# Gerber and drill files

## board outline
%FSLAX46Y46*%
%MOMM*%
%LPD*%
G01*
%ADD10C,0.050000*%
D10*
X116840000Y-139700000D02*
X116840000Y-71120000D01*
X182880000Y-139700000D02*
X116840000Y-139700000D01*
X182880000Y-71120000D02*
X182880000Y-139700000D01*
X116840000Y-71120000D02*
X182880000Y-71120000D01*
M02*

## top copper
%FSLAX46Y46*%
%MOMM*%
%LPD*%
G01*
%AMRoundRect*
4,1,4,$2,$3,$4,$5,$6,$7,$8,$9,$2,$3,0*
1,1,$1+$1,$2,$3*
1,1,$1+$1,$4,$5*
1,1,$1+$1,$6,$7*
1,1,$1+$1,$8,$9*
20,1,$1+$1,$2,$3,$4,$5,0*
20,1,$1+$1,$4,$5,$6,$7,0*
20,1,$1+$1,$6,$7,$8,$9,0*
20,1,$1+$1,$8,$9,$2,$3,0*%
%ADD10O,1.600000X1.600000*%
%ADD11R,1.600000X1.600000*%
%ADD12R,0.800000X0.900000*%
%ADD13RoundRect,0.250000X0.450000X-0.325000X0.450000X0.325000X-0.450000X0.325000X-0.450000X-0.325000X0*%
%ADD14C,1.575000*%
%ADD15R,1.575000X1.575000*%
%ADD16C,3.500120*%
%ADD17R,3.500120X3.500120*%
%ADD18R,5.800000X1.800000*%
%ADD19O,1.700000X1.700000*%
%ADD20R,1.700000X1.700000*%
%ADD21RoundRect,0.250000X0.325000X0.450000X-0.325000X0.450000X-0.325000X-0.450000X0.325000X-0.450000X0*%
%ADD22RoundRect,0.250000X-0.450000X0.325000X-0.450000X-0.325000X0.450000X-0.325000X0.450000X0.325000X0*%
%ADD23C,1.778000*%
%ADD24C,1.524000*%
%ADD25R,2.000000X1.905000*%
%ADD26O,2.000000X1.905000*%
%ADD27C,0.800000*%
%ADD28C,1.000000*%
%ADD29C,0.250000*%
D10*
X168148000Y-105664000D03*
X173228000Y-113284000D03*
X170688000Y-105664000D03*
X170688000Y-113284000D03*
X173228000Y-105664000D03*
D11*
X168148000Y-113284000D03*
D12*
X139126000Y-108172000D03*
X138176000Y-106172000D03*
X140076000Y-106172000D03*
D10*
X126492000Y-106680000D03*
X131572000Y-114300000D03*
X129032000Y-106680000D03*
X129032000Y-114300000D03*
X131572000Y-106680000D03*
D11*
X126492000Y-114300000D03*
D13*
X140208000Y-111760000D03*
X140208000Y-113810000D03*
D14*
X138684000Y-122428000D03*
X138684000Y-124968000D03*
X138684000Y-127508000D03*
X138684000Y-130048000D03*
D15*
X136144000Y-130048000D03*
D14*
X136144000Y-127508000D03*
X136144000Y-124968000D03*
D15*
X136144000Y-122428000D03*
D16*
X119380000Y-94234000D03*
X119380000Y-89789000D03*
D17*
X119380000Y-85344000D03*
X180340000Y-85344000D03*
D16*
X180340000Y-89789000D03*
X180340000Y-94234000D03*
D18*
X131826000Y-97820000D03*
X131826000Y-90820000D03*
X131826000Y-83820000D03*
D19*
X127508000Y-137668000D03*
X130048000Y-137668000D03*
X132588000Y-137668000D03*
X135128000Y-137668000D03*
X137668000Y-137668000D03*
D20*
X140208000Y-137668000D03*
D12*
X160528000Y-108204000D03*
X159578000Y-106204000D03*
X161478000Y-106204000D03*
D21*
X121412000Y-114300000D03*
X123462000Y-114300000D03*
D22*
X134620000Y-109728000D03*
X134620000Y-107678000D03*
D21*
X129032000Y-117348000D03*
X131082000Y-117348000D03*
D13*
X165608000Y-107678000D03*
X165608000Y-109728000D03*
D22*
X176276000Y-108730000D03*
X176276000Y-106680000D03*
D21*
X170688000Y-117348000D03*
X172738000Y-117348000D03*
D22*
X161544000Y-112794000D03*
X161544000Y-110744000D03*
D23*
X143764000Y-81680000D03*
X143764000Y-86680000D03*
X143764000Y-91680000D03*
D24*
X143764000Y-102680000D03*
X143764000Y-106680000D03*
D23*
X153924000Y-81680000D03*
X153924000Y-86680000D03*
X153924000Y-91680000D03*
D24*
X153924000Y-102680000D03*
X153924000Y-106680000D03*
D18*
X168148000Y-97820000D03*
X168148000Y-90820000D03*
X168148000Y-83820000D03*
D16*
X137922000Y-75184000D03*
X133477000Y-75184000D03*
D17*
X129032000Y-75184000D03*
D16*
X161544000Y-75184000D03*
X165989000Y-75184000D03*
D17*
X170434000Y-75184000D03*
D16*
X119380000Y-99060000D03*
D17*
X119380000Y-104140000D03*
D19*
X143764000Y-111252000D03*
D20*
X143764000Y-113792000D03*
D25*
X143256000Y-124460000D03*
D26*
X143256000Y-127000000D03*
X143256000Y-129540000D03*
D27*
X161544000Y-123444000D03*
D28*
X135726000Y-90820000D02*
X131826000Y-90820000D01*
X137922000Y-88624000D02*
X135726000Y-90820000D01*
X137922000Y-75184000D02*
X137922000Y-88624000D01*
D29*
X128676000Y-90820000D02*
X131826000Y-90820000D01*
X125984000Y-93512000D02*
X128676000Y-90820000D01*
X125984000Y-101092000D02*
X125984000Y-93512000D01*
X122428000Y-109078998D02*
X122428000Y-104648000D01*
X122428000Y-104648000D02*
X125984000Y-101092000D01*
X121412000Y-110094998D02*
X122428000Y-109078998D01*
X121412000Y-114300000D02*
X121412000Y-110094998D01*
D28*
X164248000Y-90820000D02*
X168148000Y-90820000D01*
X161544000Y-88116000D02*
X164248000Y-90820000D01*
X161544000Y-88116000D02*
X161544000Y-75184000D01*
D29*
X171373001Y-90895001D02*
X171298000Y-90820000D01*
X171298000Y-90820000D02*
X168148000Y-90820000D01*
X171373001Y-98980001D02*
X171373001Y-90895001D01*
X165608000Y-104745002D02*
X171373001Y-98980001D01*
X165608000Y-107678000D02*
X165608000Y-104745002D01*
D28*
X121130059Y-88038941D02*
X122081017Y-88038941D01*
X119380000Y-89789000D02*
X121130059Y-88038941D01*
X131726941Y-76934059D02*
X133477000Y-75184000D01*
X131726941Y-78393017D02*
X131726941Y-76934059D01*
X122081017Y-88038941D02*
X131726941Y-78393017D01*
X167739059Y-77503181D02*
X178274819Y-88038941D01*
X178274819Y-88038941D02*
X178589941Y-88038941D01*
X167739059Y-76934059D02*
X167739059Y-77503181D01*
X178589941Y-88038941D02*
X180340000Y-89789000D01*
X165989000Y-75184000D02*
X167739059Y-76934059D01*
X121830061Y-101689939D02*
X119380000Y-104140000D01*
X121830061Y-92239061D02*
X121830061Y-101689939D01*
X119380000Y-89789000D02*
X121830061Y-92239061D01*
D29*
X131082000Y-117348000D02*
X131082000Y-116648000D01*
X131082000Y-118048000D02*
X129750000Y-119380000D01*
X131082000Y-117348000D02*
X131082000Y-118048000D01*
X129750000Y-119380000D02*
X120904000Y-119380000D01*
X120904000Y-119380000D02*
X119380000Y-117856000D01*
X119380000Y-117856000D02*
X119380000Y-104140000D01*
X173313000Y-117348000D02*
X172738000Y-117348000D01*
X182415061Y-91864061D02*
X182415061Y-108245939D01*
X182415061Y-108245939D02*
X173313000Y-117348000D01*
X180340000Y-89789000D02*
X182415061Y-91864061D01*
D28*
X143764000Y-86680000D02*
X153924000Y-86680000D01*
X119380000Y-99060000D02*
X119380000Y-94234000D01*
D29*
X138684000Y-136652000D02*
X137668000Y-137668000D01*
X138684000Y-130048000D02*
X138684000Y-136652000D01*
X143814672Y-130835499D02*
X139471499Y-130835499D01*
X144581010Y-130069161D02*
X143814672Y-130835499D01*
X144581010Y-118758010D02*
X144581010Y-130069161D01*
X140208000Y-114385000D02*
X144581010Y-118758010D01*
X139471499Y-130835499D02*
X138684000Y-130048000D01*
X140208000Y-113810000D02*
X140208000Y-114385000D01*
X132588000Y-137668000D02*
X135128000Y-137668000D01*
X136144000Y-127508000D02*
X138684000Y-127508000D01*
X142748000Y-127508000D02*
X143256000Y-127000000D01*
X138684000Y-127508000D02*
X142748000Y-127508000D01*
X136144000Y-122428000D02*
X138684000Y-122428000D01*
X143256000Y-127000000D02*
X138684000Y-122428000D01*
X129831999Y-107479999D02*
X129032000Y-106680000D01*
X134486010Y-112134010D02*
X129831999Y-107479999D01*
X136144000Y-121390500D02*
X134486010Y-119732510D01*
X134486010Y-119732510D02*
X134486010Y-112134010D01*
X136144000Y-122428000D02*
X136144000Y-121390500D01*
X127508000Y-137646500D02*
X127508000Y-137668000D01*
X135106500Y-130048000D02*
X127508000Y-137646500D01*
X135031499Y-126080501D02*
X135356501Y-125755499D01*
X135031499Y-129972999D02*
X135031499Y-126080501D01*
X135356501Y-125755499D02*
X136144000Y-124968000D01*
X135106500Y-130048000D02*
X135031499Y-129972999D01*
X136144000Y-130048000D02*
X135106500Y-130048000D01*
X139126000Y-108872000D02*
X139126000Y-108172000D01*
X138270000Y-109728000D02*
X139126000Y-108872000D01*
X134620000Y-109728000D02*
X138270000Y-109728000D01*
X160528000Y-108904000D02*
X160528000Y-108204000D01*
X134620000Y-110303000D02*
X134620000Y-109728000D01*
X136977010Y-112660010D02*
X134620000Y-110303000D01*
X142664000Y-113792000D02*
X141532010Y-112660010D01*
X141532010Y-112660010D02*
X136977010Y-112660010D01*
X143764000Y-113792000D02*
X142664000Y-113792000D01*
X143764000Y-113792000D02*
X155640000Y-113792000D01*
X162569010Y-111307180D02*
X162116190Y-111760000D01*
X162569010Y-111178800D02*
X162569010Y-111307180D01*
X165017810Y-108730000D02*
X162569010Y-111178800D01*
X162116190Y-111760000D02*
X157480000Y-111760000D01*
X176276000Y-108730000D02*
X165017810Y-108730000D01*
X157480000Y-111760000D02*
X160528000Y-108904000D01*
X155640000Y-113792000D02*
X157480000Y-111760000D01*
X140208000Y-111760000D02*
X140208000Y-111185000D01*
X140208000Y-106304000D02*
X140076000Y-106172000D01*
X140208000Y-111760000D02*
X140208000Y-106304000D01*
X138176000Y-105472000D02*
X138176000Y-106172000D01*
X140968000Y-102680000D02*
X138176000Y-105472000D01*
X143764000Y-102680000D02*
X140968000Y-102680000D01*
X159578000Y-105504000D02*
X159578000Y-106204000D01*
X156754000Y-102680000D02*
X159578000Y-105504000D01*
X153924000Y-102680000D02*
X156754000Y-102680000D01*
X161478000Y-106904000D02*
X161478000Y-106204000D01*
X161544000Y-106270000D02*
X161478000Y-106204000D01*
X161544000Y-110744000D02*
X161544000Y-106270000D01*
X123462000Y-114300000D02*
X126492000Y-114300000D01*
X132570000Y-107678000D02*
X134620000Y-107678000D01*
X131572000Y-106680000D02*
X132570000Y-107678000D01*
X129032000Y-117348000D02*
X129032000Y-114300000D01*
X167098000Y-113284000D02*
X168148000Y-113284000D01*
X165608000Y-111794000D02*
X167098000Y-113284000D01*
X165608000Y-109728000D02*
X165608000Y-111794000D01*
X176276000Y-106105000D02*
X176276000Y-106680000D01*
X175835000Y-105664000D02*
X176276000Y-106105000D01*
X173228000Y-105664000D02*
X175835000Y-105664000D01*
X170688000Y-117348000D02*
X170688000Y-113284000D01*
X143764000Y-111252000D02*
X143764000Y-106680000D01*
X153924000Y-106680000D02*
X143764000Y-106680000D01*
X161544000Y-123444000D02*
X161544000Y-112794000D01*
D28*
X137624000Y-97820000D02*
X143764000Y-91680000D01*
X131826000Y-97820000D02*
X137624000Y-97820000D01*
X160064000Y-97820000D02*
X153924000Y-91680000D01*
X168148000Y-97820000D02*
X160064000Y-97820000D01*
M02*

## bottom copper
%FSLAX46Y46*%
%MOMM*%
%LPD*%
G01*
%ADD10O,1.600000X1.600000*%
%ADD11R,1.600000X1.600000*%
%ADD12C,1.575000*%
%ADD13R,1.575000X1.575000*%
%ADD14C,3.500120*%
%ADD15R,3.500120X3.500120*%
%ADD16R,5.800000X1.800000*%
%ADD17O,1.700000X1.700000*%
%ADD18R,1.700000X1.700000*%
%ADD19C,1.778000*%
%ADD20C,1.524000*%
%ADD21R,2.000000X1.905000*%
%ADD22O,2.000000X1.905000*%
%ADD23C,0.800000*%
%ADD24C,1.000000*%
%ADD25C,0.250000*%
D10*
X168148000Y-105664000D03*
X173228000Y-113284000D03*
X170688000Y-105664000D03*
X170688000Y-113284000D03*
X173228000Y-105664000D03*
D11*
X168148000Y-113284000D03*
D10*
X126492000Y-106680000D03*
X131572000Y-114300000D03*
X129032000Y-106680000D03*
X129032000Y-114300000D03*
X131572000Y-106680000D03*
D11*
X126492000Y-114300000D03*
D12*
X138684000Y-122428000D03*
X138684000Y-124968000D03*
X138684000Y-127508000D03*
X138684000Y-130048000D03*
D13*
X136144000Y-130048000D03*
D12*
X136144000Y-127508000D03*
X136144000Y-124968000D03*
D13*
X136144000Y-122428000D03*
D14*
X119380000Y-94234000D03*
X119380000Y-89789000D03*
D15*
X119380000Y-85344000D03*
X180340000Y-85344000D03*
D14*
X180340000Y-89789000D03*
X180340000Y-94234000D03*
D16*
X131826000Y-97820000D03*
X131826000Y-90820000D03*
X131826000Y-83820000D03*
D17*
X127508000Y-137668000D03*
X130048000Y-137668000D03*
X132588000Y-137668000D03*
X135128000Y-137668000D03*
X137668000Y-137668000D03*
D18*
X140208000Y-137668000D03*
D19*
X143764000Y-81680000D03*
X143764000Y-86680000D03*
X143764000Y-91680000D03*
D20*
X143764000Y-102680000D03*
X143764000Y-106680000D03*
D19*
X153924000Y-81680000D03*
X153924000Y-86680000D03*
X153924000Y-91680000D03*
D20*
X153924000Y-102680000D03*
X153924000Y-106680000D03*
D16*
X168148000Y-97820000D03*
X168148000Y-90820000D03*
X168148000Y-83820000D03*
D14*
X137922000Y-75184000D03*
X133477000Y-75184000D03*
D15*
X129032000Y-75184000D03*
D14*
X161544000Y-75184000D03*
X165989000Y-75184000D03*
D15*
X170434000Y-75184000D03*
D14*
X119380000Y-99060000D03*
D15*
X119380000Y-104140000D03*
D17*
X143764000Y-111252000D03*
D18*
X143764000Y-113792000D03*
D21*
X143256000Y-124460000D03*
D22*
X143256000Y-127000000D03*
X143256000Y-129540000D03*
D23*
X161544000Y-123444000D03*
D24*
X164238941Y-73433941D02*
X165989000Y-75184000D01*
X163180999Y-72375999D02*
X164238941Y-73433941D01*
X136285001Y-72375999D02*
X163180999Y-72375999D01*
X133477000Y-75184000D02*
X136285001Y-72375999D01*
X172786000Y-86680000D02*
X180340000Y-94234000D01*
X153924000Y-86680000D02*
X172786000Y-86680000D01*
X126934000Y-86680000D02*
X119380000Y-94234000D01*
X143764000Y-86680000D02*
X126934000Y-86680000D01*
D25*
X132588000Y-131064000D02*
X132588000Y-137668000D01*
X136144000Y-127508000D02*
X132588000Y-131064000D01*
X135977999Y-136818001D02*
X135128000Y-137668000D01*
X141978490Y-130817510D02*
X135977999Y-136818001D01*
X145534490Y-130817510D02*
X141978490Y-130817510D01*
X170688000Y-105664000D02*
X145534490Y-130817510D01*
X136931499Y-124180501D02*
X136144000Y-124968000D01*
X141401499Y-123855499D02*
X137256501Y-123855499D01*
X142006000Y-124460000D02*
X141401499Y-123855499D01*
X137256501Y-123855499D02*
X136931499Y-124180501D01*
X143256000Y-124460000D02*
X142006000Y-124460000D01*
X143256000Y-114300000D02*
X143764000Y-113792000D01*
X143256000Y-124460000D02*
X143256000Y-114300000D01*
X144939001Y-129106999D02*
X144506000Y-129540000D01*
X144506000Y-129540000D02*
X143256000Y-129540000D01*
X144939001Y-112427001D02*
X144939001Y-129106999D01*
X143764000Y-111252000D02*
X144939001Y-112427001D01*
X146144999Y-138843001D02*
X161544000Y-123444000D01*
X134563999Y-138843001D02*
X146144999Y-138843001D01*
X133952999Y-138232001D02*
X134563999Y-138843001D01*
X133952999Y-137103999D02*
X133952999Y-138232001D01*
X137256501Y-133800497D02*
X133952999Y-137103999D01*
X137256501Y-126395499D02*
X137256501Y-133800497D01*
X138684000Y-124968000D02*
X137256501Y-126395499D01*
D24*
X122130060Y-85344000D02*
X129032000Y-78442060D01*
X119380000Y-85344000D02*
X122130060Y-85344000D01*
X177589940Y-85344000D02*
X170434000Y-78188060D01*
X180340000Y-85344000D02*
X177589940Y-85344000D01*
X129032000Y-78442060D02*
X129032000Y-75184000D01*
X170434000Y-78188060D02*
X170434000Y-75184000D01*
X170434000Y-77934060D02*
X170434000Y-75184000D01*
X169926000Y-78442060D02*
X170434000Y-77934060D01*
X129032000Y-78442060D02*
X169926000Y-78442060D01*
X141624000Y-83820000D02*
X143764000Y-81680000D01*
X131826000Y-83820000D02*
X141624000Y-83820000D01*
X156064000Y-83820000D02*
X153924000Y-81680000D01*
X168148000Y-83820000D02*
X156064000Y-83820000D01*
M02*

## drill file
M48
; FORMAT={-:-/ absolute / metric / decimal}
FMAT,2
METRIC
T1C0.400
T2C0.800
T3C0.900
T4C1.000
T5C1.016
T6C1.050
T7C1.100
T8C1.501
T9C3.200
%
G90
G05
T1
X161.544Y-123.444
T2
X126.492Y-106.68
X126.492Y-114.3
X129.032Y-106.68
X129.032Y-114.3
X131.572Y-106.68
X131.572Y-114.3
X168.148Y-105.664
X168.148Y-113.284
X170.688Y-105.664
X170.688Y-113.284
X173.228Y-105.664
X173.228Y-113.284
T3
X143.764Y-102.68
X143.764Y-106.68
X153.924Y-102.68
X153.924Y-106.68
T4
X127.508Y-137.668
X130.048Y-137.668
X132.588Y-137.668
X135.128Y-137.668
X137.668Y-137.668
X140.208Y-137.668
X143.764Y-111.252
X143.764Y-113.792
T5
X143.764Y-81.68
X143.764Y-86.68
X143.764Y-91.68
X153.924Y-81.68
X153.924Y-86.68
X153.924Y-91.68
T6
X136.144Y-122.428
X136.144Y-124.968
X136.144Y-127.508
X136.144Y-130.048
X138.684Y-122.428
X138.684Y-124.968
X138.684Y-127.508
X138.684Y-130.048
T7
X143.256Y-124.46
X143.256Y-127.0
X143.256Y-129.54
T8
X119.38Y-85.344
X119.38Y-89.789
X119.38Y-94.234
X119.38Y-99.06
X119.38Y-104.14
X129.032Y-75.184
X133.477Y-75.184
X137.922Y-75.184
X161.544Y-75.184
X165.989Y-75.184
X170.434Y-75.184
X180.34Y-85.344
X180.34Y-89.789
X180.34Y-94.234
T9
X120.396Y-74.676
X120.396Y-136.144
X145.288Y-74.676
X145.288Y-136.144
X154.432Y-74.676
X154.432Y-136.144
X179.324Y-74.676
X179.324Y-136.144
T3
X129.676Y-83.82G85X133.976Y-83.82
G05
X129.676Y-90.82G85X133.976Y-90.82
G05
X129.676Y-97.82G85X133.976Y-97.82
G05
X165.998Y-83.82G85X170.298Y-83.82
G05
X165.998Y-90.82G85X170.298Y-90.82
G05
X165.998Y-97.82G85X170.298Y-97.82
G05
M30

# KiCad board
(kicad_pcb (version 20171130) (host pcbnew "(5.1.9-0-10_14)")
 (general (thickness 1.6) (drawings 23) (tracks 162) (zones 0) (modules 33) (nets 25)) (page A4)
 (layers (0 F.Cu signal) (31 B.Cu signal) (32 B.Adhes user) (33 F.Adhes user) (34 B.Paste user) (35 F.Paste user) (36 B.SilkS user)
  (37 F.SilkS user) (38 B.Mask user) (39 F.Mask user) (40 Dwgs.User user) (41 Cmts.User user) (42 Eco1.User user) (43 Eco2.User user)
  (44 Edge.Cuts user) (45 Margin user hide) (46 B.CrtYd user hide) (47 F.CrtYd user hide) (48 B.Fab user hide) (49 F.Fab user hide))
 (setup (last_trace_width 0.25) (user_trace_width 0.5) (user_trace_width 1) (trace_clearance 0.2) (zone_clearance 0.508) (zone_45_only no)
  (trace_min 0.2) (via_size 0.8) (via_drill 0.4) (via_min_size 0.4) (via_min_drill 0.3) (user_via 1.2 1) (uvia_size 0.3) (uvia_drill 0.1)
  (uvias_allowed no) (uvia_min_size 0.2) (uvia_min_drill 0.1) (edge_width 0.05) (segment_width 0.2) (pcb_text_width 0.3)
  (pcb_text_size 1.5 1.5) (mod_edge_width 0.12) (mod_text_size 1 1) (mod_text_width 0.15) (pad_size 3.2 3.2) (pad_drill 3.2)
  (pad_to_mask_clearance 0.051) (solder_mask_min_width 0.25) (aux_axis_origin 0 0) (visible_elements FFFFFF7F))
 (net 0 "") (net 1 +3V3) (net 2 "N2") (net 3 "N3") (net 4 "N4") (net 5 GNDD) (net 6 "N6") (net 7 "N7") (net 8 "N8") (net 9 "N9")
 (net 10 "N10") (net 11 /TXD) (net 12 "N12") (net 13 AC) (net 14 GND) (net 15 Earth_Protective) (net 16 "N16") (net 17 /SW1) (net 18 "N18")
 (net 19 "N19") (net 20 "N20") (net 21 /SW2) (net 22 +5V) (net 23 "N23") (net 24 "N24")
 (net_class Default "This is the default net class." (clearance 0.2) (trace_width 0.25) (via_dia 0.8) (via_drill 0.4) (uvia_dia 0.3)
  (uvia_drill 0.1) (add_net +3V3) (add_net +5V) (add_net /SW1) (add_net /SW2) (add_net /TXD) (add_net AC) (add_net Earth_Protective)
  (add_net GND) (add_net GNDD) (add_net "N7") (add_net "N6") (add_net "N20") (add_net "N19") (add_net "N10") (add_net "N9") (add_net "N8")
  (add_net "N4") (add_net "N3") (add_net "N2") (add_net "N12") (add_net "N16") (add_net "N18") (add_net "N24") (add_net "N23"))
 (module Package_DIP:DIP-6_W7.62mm (layer F.Cu) (at 168.148 113.284 90)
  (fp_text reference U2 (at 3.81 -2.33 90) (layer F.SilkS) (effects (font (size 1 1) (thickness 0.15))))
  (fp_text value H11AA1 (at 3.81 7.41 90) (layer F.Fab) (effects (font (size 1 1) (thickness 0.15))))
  (pad 6 thru_hole oval (at 7.62 0 90) (size 1.6 1.6) (drill 0.8) (layers *.Cu *.Mask))
  (pad 3 thru_hole oval (at 0 5.08 90) (size 1.6 1.6) (drill 0.8) (layers *.Cu *.Mask))
  (pad 5 thru_hole oval (at 7.62 2.54 90) (size 1.6 1.6) (drill 0.8) (layers *.Cu *.Mask) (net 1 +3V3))
  (pad 2 thru_hole oval (at 0 2.54 90) (size 1.6 1.6) (drill 0.8) (layers *.Cu *.Mask) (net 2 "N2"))
  (pad 4 thru_hole oval (at 7.62 5.08 90) (size 1.6 1.6) (drill 0.8) (layers *.Cu *.Mask) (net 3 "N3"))
  (pad 1 thru_hole rect (at 0 0 90) (size 1.6 1.6) (drill 0.8) (layers *.Cu *.Mask) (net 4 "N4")))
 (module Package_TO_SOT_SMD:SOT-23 (layer F.Cu) (at 139.126 107.172 270)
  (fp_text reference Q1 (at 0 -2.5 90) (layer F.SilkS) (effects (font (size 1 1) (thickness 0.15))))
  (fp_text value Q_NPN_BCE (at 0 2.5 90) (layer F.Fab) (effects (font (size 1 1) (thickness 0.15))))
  (pad 3 smd rect (at 1 0 270) (size 0.9 0.8) (layers F.Cu F.Paste F.Mask) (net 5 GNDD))
  (pad 2 smd rect (at -1 0.95 270) (size 0.9 0.8) (layers F.Cu F.Paste F.Mask) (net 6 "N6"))
  (pad 1 smd rect (at -1 -0.95 270) (size 0.9 0.8) (layers F.Cu F.Paste F.Mask) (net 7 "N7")))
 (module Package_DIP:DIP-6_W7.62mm (layer F.Cu) (at 126.492 114.3 90)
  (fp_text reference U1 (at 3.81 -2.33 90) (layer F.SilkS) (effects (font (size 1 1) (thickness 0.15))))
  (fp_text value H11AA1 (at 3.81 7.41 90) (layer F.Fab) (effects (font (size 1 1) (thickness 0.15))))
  (pad 6 thru_hole oval (at 7.62 0 90) (size 1.6 1.6) (drill 0.8) (layers *.Cu *.Mask))
  (pad 3 thru_hole oval (at 0 5.08 90) (size 1.6 1.6) (drill 0.8) (layers *.Cu *.Mask))
  (pad 5 thru_hole oval (at 7.62 2.54 90) (size 1.6 1.6) (drill 0.8) (layers *.Cu *.Mask) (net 1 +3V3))
  (pad 2 thru_hole oval (at 0 2.54 90) (size 1.6 1.6) (drill 0.8) (layers *.Cu *.Mask) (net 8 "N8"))
  (pad 4 thru_hole oval (at 7.62 5.08 90) (size 1.6 1.6) (drill 0.8) (layers *.Cu *.Mask) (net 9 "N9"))
  (pad 1 thru_hole rect (at 0 0 90) (size 1.6 1.6) (drill 0.8) (layers *.Cu *.Mask) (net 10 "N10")))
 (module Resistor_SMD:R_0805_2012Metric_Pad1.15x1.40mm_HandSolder (layer F.Cu) (at 140.208 112.785 90)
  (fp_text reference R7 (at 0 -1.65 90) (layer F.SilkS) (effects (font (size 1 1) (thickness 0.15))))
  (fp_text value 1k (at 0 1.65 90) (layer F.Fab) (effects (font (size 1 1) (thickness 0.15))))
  (pad 2 smd roundrect (at 1.025 0 90) (size 1.15 1.4) (layers F.Cu F.Paste F.Mask) (roundrect_rratio 0.217391) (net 7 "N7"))
  (pad 1 smd roundrect (at -1.025 0 90) (size 1.15 1.4) (layers F.Cu F.Paste F.Mask) (roundrect_rratio 0.217391) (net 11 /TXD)))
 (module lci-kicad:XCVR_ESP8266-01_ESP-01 (layer F.Cu) (at 136.144 126.238 180)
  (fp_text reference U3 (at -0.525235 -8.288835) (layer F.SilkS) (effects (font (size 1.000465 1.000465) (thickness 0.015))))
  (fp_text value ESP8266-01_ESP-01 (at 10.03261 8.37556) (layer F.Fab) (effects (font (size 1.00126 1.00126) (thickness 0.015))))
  (pad 8 thru_hole circle (at -2.54 3.81 180) (size 1.575 1.575) (drill 1.05) (layers *.Cu *.Mask) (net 1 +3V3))
  (pad 7 thru_hole circle (at -2.54 1.27 180) (size 1.575 1.575) (drill 1.05) (layers *.Cu *.Mask) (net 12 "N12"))
  (pad 6 thru_hole circle (at -2.54 -1.27 180) (size 1.575 1.575) (drill 1.05) (layers *.Cu *.Mask) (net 1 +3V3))
  (pad 5 thru_hole circle (at -2.54 -3.81 180) (size 1.575 1.575) (drill 1.05) (layers *.Cu *.Mask) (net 11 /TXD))
  (pad 4 thru_hole rect (at 0 -3.81 180) (size 1.575 1.575) (drill 1.05) (layers *.Cu *.Mask) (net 5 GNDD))
  (pad 3 thru_hole circle (at 0 -1.27 180) (size 1.575 1.575) (drill 1.05) (layers *.Cu *.Mask) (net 1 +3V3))
  (pad 2 thru_hole circle (at 0 1.27 180) (size 1.575 1.575) (drill 1.05) (layers *.Cu *.Mask) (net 5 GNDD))
  (pad 1 thru_hole rect (at 0 3.81 180) (size 1.575 1.575) (drill 1.05) (layers *.Cu *.Mask) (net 1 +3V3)))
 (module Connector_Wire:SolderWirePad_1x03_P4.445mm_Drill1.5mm (layer F.Cu) (at 119.38 85.344 270)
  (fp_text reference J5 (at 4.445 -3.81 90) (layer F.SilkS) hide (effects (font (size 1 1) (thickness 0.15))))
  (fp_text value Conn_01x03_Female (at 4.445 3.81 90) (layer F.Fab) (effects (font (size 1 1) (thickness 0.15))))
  (pad 3 thru_hole circle (at 8.89 0 270) (size 3.50012 3.50012) (drill 1.50114) (layers *.Cu *.Mask) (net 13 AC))
  (pad 2 thru_hole circle (at 4.445 0 270) (size 3.50012 3.50012) (drill 1.50114) (layers *.Cu *.Mask) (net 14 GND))
  (pad 1 thru_hole rect (at 0 0 270) (size 3.50012 3.50012) (drill 1.50114) (layers *.Cu *.Mask) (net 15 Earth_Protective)))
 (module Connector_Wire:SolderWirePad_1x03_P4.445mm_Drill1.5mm (layer F.Cu) (at 180.34 85.344 270)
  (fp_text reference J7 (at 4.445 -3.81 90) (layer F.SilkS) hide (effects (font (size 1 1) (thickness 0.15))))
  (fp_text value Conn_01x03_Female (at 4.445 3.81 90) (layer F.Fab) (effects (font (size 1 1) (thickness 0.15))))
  (pad 1 thru_hole rect (at 0 0 270) (size 3.50012 3.50012) (drill 1.50114) (layers *.Cu *.Mask) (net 15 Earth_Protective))
  (pad 2 thru_hole circle (at 4.445 0 270) (size 3.50012 3.50012) (drill 1.50114) (layers *.Cu *.Mask) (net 14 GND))
  (pad 3 thru_hole circle (at 8.89 0 270) (size 3.50012 3.50012) (drill 1.50114) (layers *.Cu *.Mask) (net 13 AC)))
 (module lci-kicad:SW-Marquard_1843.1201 (layer F.Cu) (at 131.572 90.932)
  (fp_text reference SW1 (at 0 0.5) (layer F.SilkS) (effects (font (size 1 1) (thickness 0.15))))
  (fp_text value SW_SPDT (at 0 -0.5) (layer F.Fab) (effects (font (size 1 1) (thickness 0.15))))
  (pad 3 thru_hole rect (at 0.254 6.888) (size 5.8 1.8) (drill oval 5.2 0.9) (layers *.Cu *.Mask) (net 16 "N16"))
  (pad 2 thru_hole rect (at 0.254 -0.112) (size 5.8 1.8) (drill oval 5.2 0.9) (layers *.Cu *.Mask) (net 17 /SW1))
  (pad 1 thru_hole rect (at 0.254 -7.112) (size 5.8 1.8) (drill oval 5.2 0.9) (layers *.Cu *.Mask) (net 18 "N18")))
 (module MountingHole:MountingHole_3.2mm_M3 (layer F.Cu) (at 120.396 74.676)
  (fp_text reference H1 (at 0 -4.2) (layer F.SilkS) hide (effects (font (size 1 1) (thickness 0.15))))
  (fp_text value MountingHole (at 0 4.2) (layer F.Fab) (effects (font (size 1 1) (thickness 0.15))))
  (pad 1 np_thru_hole circle (at 0 0) (size 3.2 3.2) (drill 3.2) (layers *.Cu *.Mask)))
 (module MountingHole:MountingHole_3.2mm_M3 (layer F.Cu) (at 120.396 136.144)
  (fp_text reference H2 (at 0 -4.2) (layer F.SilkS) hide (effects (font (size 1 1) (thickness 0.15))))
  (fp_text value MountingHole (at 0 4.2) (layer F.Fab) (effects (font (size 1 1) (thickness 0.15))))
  (pad 1 np_thru_hole circle (at 0 0) (size 3.2 3.2) (drill 3.2) (layers *.Cu *.Mask)))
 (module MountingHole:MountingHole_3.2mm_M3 (layer F.Cu) (at 179.324 74.676)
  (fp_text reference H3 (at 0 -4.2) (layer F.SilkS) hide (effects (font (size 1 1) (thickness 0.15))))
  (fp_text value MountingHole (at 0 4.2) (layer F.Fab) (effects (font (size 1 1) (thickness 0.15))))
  (pad 1 np_thru_hole circle (at 0 0) (size 3.2 3.2) (drill 3.2) (layers *.Cu *.Mask)))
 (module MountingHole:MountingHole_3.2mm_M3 (layer F.Cu) (at 179.324 136.144)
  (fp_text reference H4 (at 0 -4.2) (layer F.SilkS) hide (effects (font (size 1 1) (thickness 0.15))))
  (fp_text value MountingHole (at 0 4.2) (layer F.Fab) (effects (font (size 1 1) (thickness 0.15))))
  (pad "" np_thru_hole circle (at 0 0) (size 3.2 3.2) (drill 3.2) (layers *.Cu *.Mask)))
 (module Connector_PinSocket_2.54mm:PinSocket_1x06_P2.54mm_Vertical (layer F.Cu) (at 140.208 137.668 270)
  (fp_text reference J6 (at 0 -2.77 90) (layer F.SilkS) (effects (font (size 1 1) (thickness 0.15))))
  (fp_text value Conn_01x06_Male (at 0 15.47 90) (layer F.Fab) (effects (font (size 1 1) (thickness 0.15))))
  (pad 6 thru_hole oval (at 0 12.7 270) (size 1.7 1.7) (drill 1) (layers *.Cu *.Mask) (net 5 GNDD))
  (pad 5 thru_hole oval (at 0 10.16 270) (size 1.7 1.7) (drill 1) (layers *.Cu *.Mask))
  (pad 4 thru_hole oval (at 0 7.62 270) (size 1.7 1.7) (drill 1) (layers *.Cu *.Mask) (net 1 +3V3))
  (pad 3 thru_hole oval (at 0 5.08 270) (size 1.7 1.7) (drill 1) (layers *.Cu *.Mask) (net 1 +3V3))
  (pad 2 thru_hole oval (at 0 2.54 270) (size 1.7 1.7) (drill 1) (layers *.Cu *.Mask) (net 11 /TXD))
  (pad 1 thru_hole rect (at 0 0 270) (size 1.7 1.7) (drill 1) (layers *.Cu *.Mask)))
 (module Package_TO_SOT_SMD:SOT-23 (layer F.Cu) (at 160.528 107.204 270)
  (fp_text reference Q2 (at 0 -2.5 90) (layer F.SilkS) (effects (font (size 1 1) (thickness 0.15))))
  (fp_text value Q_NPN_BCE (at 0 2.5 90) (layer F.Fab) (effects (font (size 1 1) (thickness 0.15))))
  (pad 3 smd rect (at 1 0 270) (size 0.9 0.8) (layers F.Cu F.Paste F.Mask) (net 5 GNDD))
  (pad 2 smd rect (at -1 0.95 270) (size 0.9 0.8) (layers F.Cu F.Paste F.Mask) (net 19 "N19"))
  (pad 1 smd rect (at -1 -0.95 270) (size 0.9 0.8) (layers F.Cu F.Paste F.Mask) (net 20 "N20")))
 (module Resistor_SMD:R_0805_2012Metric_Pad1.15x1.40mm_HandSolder (layer F.Cu) (at 122.437 114.3 180)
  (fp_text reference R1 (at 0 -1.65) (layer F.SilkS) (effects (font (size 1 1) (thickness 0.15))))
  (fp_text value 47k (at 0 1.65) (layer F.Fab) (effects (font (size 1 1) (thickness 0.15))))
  (pad 2 smd roundrect (at 1.025 0 180) (size 1.15 1.4) (layers F.Cu F.Paste F.Mask) (roundrect_rratio 0.217391) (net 17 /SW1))
  (pad 1 smd roundrect (at -1.025 0 180) (size 1.15 1.4) (layers F.Cu F.Paste F.Mask) (roundrect_rratio 0.217391) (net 10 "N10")))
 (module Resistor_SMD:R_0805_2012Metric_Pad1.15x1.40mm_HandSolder (layer F.Cu) (at 134.62 108.703 270)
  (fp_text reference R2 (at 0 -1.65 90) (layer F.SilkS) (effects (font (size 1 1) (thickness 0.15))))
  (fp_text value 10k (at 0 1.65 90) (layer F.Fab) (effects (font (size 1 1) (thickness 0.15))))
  (pad 2 smd roundrect (at 1.025 0 270) (size 1.15 1.4) (layers F.Cu F.Paste F.Mask) (roundrect_rratio 0.217391) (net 5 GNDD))
  (pad 1 smd roundrect (at -1.025 0 270) (size 1.15 1.4) (layers F.Cu F.Paste F.Mask) (roundrect_rratio 0.217391) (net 9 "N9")))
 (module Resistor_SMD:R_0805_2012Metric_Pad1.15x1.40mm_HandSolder (layer F.Cu) (at 130.057 117.348 180)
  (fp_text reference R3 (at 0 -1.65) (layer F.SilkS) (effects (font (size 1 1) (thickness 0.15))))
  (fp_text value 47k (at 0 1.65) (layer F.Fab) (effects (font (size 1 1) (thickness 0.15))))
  (pad 2 smd roundrect (at 1.025 0 180) (size 1.15 1.4) (layers F.Cu F.Paste F.Mask) (roundrect_rratio 0.217391) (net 8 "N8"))
  (pad 1 smd roundrect (at -1.025 0 180) (size 1.15 1.4) (layers F.Cu F.Paste F.Mask) (roundrect_rratio 0.217391) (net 14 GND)))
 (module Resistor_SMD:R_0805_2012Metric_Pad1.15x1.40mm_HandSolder (layer F.Cu) (at 165.608 108.703 90)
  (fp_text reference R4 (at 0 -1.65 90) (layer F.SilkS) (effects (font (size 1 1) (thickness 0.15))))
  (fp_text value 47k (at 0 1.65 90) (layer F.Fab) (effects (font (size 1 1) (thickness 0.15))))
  (pad 2 smd roundrect (at 1.025 0 90) (size 1.15 1.4) (layers F.Cu F.Paste F.Mask) (roundrect_rratio 0.217391) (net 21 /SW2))
  (pad 1 smd roundrect (at -1.025 0 90) (size 1.15 1.4) (layers F.Cu F.Paste F.Mask) (roundrect_rratio 0.217391) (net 4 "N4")))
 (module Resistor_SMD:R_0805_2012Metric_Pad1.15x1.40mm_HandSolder (layer F.Cu) (at 176.276 107.705 270)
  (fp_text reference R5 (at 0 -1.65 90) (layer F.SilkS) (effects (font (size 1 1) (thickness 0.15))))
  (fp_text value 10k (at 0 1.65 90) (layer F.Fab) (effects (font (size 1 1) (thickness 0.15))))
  (pad 2 smd roundrect (at 1.025 0 270) (size 1.15 1.4) (layers F.Cu F.Paste F.Mask) (roundrect_rratio 0.217391) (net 5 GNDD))
  (pad 1 smd roundrect (at -1.025 0 270) (size 1.15 1.4) (layers F.Cu F.Paste F.Mask) (roundrect_rratio 0.217391) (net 3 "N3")))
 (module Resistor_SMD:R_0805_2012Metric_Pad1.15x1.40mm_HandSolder (layer F.Cu) (at 171.713 117.348 180)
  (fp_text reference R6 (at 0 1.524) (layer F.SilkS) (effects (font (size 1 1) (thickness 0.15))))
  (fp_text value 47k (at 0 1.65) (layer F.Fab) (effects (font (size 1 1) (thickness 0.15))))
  (pad 2 smd roundrect (at 1.025 0 180) (size 1.15 1.4) (layers F.Cu F.Paste F.Mask) (roundrect_rratio 0.217391) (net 2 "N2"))
  (pad 1 smd roundrect (at -1.025 0 180) (size 1.15 1.4) (layers F.Cu F.Paste F.Mask) (roundrect_rratio 0.217391) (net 14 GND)))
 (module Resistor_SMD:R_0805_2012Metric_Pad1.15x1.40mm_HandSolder (layer F.Cu) (at 161.544 111.769 270)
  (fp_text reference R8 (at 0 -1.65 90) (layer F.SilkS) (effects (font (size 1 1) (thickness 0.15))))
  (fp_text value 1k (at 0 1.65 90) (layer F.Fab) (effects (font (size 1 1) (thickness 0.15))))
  (pad 2 smd roundrect (at 1.025 0 270) (size 1.15 1.4) (layers F.Cu F.Paste F.Mask) (roundrect_rratio 0.217391) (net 12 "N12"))
  (pad 1 smd roundrect (at -1.025 0 270) (size 1.15 1.4) (layers F.Cu F.Paste F.Mask) (roundrect_rratio 0.217391) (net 20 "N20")))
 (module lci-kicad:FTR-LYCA (layer F.Cu) (at 143.764 106.68 90)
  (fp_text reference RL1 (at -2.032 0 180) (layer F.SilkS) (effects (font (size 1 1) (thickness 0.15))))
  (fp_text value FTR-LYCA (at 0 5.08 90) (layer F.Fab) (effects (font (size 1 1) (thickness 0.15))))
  (pad 5 thru_hole circle (at 25 0 90) (size 1.778 1.778) (drill 1.016) (layers *.Cu *.Mask) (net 18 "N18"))
  (pad 4 thru_hole circle (at 20 0 90) (size 1.778 1.778) (drill 1.016) (layers *.Cu *.Mask) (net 13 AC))
  (pad 3 thru_hole circle (at 15 0 90) (size 1.778 1.778) (drill 1.016) (layers *.Cu *.Mask) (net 16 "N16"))
  (pad 2 thru_hole circle (at 4 0 90) (size 1.524 1.524) (drill 0.9) (layers *.Cu *.Mask) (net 6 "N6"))
  (pad 1 thru_hole circle (at 0 0 90) (size 1.524 1.524) (drill 0.9) (layers *.Cu *.Mask) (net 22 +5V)))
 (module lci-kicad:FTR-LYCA (layer F.Cu) (at 153.924 106.68 90)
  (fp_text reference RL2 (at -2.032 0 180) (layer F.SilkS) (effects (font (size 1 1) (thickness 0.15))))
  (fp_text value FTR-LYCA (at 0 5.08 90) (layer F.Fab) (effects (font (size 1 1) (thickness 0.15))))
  (pad 5 thru_hole circle (at 25 0 90) (size 1.778 1.778) (drill 1.016) (layers *.Cu *.Mask) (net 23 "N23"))
  (pad 4 thru_hole circle (at 20 0 90) (size 1.778 1.778) (drill 1.016) (layers *.Cu *.Mask) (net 13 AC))
  (pad 3 thru_hole circle (at 15 0 90) (size 1.778 1.778) (drill 1.016) (layers *.Cu *.Mask) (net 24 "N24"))
  (pad 2 thru_hole circle (at 4 0 90) (size 1.524 1.524) (drill 0.9) (layers *.Cu *.Mask) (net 19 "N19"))
  (pad 1 thru_hole circle (at 0 0 90) (size 1.524 1.524) (drill 0.9) (layers *.Cu *.Mask) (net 22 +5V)))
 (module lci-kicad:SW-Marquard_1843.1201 (layer F.Cu) (at 167.894 90.932)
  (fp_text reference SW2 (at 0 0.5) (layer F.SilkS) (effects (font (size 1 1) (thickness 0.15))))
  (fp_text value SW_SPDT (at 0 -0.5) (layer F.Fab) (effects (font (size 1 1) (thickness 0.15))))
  (pad 3 thru_hole rect (at 0.254 6.888) (size 5.8 1.8) (drill oval 5.2 0.9) (layers *.Cu *.Mask) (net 24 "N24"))
  (pad 2 thru_hole rect (at 0.254 -0.112) (size 5.8 1.8) (drill oval 5.2 0.9) (layers *.Cu *.Mask) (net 21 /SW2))
  (pad 1 thru_hole rect (at 0.254 -7.112) (size 5.8 1.8) (drill oval 5.2 0.9) (layers *.Cu *.Mask) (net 23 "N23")))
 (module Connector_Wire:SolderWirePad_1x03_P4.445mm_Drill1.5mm (layer F.Cu) (at 129.032 75.184)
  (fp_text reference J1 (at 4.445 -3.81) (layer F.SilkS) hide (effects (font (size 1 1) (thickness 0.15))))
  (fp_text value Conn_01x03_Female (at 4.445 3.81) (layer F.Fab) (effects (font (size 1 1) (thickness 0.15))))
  (pad 3 thru_hole circle (at 8.89 0) (size 3.50012 3.50012) (drill 1.50114) (layers *.Cu *.Mask) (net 17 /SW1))
  (pad 2 thru_hole circle (at 4.445 0) (size 3.50012 3.50012) (drill 1.50114) (layers *.Cu *.Mask) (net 14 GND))
  (pad 1 thru_hole rect (at 0 0) (size 3.50012 3.50012) (drill 1.50114) (layers *.Cu *.Mask) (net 15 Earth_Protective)))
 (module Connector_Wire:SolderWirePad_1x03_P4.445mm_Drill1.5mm (layer F.Cu) (at 170.434 75.184 180)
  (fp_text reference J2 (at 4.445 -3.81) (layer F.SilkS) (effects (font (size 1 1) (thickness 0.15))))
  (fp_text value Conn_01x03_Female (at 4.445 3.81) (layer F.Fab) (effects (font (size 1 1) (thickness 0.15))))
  (pad 3 thru_hole circle (at 8.89 0 180) (size 3.50012 3.50012) (drill 1.50114) (layers *.Cu *.Mask) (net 21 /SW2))
  (pad 2 thru_hole circle (at 4.445 0 180) (size 3.50012 3.50012) (drill 1.50114) (layers *.Cu *.Mask) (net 14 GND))
  (pad 1 thru_hole rect (at 0 0 180) (size 3.50012 3.50012) (drill 1.50114) (layers *.Cu *.Mask) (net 15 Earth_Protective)))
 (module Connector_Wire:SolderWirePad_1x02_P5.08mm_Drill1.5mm (layer F.Cu) (at 119.38 104.14 90)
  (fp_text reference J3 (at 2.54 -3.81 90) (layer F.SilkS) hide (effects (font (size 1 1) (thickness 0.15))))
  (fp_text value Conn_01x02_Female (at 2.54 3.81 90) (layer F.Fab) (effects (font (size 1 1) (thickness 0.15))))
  (pad 2 thru_hole circle (at 5.08 0 90) (size 3.50012 3.50012) (drill 1.50114) (layers *.Cu *.Mask) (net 13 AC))
  (pad 1 thru_hole rect (at 0 0 90) (size 3.50012 3.50012) (drill 1.50114) (layers *.Cu *.Mask) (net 14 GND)))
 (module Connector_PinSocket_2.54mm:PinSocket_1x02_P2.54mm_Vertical (layer F.Cu) (at 143.764 113.792 180)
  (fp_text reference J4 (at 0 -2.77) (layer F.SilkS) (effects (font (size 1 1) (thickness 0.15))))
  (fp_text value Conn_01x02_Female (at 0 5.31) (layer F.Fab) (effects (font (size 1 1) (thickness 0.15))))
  (pad 2 thru_hole oval (at 0 2.54 180) (size 1.7 1.7) (drill 1) (layers *.Cu *.Mask) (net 22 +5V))
  (pad 1 thru_hole rect (at 0 0 180) (size 1.7 1.7) (drill 1) (layers *.Cu *.Mask) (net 5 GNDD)))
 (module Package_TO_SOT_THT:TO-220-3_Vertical (layer F.Cu) (at 143.256 124.46 270)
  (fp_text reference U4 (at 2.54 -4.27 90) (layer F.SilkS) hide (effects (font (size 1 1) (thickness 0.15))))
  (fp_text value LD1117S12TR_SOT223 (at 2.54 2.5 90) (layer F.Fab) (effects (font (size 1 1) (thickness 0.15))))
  (pad 1 thru_hole rect (at 0 0 270) (size 1.905 2) (drill 1.1) (layers *.Cu *.Mask) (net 5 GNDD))
  (pad 2 thru_hole oval (at 2.54 0 270) (size 1.905 2) (drill 1.1) (layers *.Cu *.Mask) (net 1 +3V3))
  (pad 3 thru_hole oval (at 5.08 0 270) (size 1.905 2) (drill 1.1) (layers *.Cu *.Mask) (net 22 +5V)))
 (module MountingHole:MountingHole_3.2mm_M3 (layer F.Cu) (at 145.288 74.676)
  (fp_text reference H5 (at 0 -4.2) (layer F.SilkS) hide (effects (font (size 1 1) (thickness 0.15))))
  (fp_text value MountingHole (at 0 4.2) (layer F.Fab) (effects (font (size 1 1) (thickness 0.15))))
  (pad 1 np_thru_hole circle (at 0 0) (size 3.2 3.2) (drill 3.2) (layers *.Cu *.Mask)))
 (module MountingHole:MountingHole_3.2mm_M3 (layer F.Cu) (at 154.432 74.676)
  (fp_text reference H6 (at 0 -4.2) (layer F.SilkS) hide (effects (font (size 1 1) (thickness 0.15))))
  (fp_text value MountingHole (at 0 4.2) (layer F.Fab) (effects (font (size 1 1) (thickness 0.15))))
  (pad 1 np_thru_hole circle (at 0 0) (size 3.2 3.2) (drill 3.2) (layers *.Cu *.Mask)))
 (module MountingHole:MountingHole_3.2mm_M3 (layer F.Cu) (at 145.288 136.144)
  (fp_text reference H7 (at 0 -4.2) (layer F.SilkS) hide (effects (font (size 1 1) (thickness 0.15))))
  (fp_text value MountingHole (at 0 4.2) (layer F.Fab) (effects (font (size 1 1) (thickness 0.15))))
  (pad 1 np_thru_hole circle (at 0 0) (size 3.2 3.2) (drill 3.2) (layers *.Cu *.Mask)))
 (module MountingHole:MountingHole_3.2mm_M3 (layer F.Cu) (at 154.432 136.144)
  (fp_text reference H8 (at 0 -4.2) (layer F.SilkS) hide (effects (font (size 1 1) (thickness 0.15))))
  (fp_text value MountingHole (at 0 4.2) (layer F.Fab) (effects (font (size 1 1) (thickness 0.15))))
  (pad 1 np_thru_hole circle (at 0 0) (size 3.2 3.2) (drill 3.2) (layers *.Cu *.Mask)))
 (gr_line (start 116.84 139.7) (end 116.84 71.12) (layer Edge.Cuts) (width 0.05))
 (gr_line (start 182.88 139.7) (end 116.84 139.7) (layer Edge.Cuts) (width 0.05))
 (gr_line (start 182.88 71.12) (end 182.88 139.7) (layer Edge.Cuts) (width 0.05))
 (gr_line (start 116.84 71.12) (end 182.88 71.12) (layer Edge.Cuts) (width 0.05))
 (segment (start 135.726 90.82) (end 131.826 90.82) (width 1) (layer F.Cu) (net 17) (status 20))
 (segment (start 137.922 88.624) (end 135.726 90.82) (width 1) (layer F.Cu) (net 17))
 (segment (start 137.922 75.184) (end 137.922 88.624) (width 1) (layer F.Cu) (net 17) (status 10))
 (segment (start 128.676 90.82) (end 131.826 90.82) (width 0.25) (layer F.Cu) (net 17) (status 20))
 (segment (start 125.984 93.512) (end 128.676 90.82) (width 0.25) (layer F.Cu) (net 17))
 (segment (start 125.984 101.092) (end 125.984 93.512) (width 0.25) (layer F.Cu) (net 17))
 (segment (start 122.428 109.078998) (end 122.428 104.648) (width 0.25) (layer F.Cu) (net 17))
 (segment (start 122.428 104.648) (end 125.984 101.092) (width 0.25) (layer F.Cu) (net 17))
 (segment (start 121.412 110.094998) (end 122.428 109.078998) (width 0.25) (layer F.Cu) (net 17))
 (segment (start 121.412 114.3) (end 121.412 110.094998) (width 0.25) (layer F.Cu) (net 17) (status 10))
 (segment (start 164.248 90.82) (end 168.148 90.82) (width 1) (layer F.Cu) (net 21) (status 20))
 (segment (start 161.544 88.116) (end 164.248 90.82) (width 1) (layer F.Cu) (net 21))
 (segment (start 161.544 88.116) (end 161.544 75.184) (width 1) (layer F.Cu) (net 21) (status 20))
 (segment (start 171.373001 90.895001) (end 171.298 90.82) (width 0.25) (layer F.Cu) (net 21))
 (segment (start 171.298 90.82) (end 168.148 90.82) (width 0.25) (layer F.Cu) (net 21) (status 20))
 (segment (start 171.373001 98.980001) (end 171.373001 90.895001) (width 0.25) (layer F.Cu) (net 21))
 (segment (start 165.608 104.745002) (end 171.373001 98.980001) (width 0.25) (layer F.Cu) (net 21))
 (segment (start 165.608 107.678) (end 165.608 104.745002) (width 0.25) (layer F.Cu) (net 21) (status 10))
 (segment (start 121.130059 88.038941) (end 122.081017 88.038941) (width 1) (layer F.Cu) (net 14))
 (segment (start 119.38 89.789) (end 121.130059 88.038941) (width 1) (layer F.Cu) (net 14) (status 10))
 (segment (start 164.238941 73.433941) (end 165.989 75.184) (width 1) (layer B.Cu) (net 14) (status 20))
 (segment (start 163.180999 72.375999) (end 164.238941 73.433941) (width 1) (layer B.Cu) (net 14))
 (segment (start 136.285001 72.375999) (end 163.180999 72.375999) (width 1) (layer B.Cu) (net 14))
 (segment (start 133.477 75.184) (end 136.285001 72.375999) (width 1) (layer B.Cu) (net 14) (status 10))
 (segment (start 131.726941 76.934059) (end 133.477 75.184) (width 1) (layer F.Cu) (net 14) (status 20))
 (segment (start 131.726941 78.393017) (end 131.726941 76.934059) (width 1) (layer F.Cu) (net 14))
 (segment (start 122.081017 88.038941) (end 131.726941 78.393017) (width 1) (layer F.Cu) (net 14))
 (segment (start 167.739059 77.503181) (end 178.274819 88.038941) (width 1) (layer F.Cu) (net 14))
 (segment (start 178.274819 88.038941) (end 178.589941 88.038941) (width 1) (layer F.Cu) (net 14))
 (segment (start 167.739059 76.934059) (end 167.739059 77.503181) (width 1) (layer F.Cu) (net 14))
 (segment (start 178.589941 88.038941) (end 180.34 89.789) (width 1) (layer F.Cu) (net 14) (status 20))
 (segment (start 165.989 75.184) (end 167.739059 76.934059) (width 1) (layer F.Cu) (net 14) (status 10))
 (segment (start 121.830061 101.689939) (end 119.38 104.14) (width 1) (layer F.Cu) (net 14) (status 20))
 (segment (start 121.830061 92.239061) (end 121.830061 101.689939) (width 1) (layer F.Cu) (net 14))
 (segment (start 119.38 89.789) (end 121.830061 92.239061) (width 1) (layer F.Cu) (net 14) (status 10))
 (segment (start 131.082 117.348) (end 131.082 116.648) (width 0.25) (layer F.Cu) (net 14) (status 30))
 (segment (start 131.082 118.048) (end 129.75 119.38) (width 0.25) (layer F.Cu) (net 14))
 (segment (start 131.082 117.348) (end 131.082 118.048) (width 0.25) (layer F.Cu) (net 14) (status 10))
 (segment (start 129.75 119.38) (end 120.904 119.38) (width 0.25) (layer F.Cu) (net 14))
 (segment (start 120.904 119.38) (end 119.38 117.856) (width 0.25) (layer F.Cu) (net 14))
 (segment (start 119.38 117.856) (end 119.38 104.14) (width 0.25) (layer F.Cu) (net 14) (status 20))
 (segment (start 173.313 117.348) (end 172.738 117.348) (width 0.25) (layer F.Cu) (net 14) (status 20))
 (segment (start 182.415061 91.864061) (end 182.415061 108.245939) (width 0.25) (layer F.Cu) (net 14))
 (segment (start 182.415061 108.245939) (end 173.313 117.348) (width 0.25) (layer F.Cu) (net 14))
 (segment (start 180.34 89.789) (end 182.415061 91.864061) (width 0.25) (layer F.Cu) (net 14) (status 10))
 (segment (start 143.764 86.68) (end 153.924 86.68) (width 1) (layer F.Cu) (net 13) (status 30))
 (segment (start 119.38 99.06) (end 119.38 94.234) (width 1) (layer F.Cu) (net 13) (status 30))
 (segment (start 172.786 86.68) (end 180.34 94.234) (width 1) (layer B.Cu) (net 13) (status 20))
 (segment (start 153.924 86.68) (end 172.786 86.68) (width 1) (layer B.Cu) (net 13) (status 10))
 (segment (start 126.934 86.68) (end 119.38 94.234) (width 1) (layer B.Cu) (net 13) (status 20))
 (segment (start 143.764 86.68) (end 126.934 86.68) (width 1) (layer B.Cu) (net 13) (status 10))
 (segment (start 138.684 136.652) (end 137.668 137.668) (width 0.25) (layer F.Cu) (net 11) (status 20))
 (segment (start 138.684 130.048) (end 138.684 136.652) (width 0.25) (layer F.Cu) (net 11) (status 10))
 (segment (start 143.814672 130.835499) (end 139.471499 130.835499) (width 0.25) (layer F.Cu) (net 11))
 (segment (start 144.58101 130.069161) (end 143.814672 130.835499) (width 0.25) (layer F.Cu) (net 11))
 (segment (start 144.58101 118.75801) (end 144.58101 130.069161) (width 0.25) (layer F.Cu) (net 11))
 (segment (start 140.208 114.385) (end 144.58101 118.75801) (width 0.25) (layer F.Cu) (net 11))
 (segment (start 139.471499 130.835499) (end 138.684 130.048) (width 0.25) (layer F.Cu) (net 11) (status 20))
 (segment (start 140.208 113.81) (end 140.208 114.385) (width 0.25) (layer F.Cu) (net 11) (status 10))
 (segment (start 132.588 137.668) (end 135.128 137.668) (width 0.25) (layer F.Cu) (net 1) (status 30))
 (segment (start 136.144 127.508) (end 138.684 127.508) (width 0.25) (layer F.Cu) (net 1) (status 30))
 (segment (start 142.748 127.508) (end 143.256 127) (width 0.25) (layer F.Cu) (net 1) (status 30))
 (segment (start 138.684 127.508) (end 142.748 127.508) (width 0.25) (layer F.Cu) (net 1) (status 30))
 (segment (start 136.144 122.428) (end 138.684 122.428) (width 0.25) (layer F.Cu) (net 1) (status 30))
 (segment (start 143.256 127) (end 138.684 122.428) (width 0.25) (layer F.Cu) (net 1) (status 30))
 (segment (start 132.588 131.064) (end 132.588 137.668) (width 0.25) (layer B.Cu) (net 1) (status 20))
 (segment (start 136.144 127.508) (end 132.588 131.064) (width 0.25) (layer B.Cu) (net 1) (status 10))
 (segment (start 129.831999 107.479999) (end 129.032 106.68) (width 0.25) (layer F.Cu) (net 1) (status 20))
 (segment (start 134.48601 112.13401) (end 129.831999 107.479999) (width 0.25) (layer F.Cu) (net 1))
 (segment (start 136.144 121.3905) (end 134.48601 119.73251) (width 0.25) (layer F.Cu) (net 1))
 (segment (start 134.48601 119.73251) (end 134.48601 112.13401) (width 0.25) (layer F.Cu) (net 1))
 (segment (start 136.144 122.428) (end 136.144 121.3905) (width 0.25) (layer F.Cu) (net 1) (status 10))
 (segment (start 135.977999 136.818001) (end 135.128 137.668) (width 0.25) (layer B.Cu) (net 1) (status 20))
 (segment (start 141.97849 130.81751) (end 135.977999 136.818001) (width 0.25) (layer B.Cu) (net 1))
 (segment (start 145.53449 130.81751) (end 141.97849 130.81751) (width 0.25) (layer B.Cu) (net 1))
 (segment (start 170.688 105.664) (end 145.53449 130.81751) (width 0.25) (layer B.Cu) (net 1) (status 10))
 (segment (start 127.508 137.6465) (end 127.508 137.668) (width 0.25) (layer F.Cu) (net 5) (status 30))
 (segment (start 135.1065 130.048) (end 127.508 137.6465) (width 0.25) (layer F.Cu) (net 5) (status 20))
 (segment (start 135.031499 126.080501) (end 135.356501 125.755499) (width 0.25) (layer F.Cu) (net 5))
 (segment (start 135.031499 129.972999) (end 135.031499 126.080501) (width 0.25) (layer F.Cu) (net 5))
 (segment (start 135.356501 125.755499) (end 136.144 124.968) (width 0.25) (layer F.Cu) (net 5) (status 20))
 (segment (start 135.1065 130.048) (end 135.031499 129.972999) (width 0.25) (layer F.Cu) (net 5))
 (segment (start 136.144 130.048) (end 135.1065 130.048) (width 0.25) (layer F.Cu) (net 5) (status 10))
 (segment (start 139.126 108.872) (end 139.126 108.172) (width 0.25) (layer F.Cu) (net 5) (status 20))
 (segment (start 138.27 109.728) (end 139.126 108.872) (width 0.25) (layer F.Cu) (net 5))
 (segment (start 134.62 109.728) (end 138.27 109.728) (width 0.25) (layer F.Cu) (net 5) (status 10))
 (segment (start 136.931499 124.180501) (end 136.144 124.968) (width 0.25) (layer B.Cu) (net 5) (status 20))
 (segment (start 141.401499 123.855499) (end 137.256501 123.855499) (width 0.25) (layer B.Cu) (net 5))
 (segment (start 142.006 124.46) (end 141.401499 123.855499) (width 0.25) (layer B.Cu) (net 5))
 (segment (start 137.256501 123.855499) (end 136.931499 124.180501) (width 0.25) (layer B.Cu) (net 5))
 (segment (start 143.256 124.46) (end 142.006 124.46) (width 0.25) (layer B.Cu) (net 5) (status 10))
 (segment (start 143.256 114.3) (end 143.764 113.792) (width 0.25) (layer B.Cu) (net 5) (status 30))
 (segment (start 143.256 124.46) (end 143.256 114.3) (width 0.25) (layer B.Cu) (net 5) (status 30))
 (segment (start 160.528 108.904) (end 160.528 108.204) (width 0.25) (layer F.Cu) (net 5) (status 20))
 (segment (start 134.62 110.303) (end 134.62 109.728) (width 0.25) (layer F.Cu) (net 5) (status 20))
 (segment (start 136.97701 112.66001) (end 134.62 110.303) (width 0.25) (layer F.Cu) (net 5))
 (segment (start 142.664 113.792) (end 141.53201 112.66001) (width 0.25) (layer F.Cu) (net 5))
 (segment (start 141.53201 112.66001) (end 136.97701 112.66001) (width 0.25) (layer F.Cu) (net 5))
 (segment (start 143.764 113.792) (end 142.664 113.792) (width 0.25) (layer F.Cu) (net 5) (status 10))
 (segment (start 143.764 113.792) (end 155.64 113.792) (width 0.25) (layer F.Cu) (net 5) (status 10))
 (segment (start 162.56901 111.30718) (end 162.11619 111.76) (width 0.25) (layer F.Cu) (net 5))
 (segment (start 162.56901 111.1788) (end 162.56901 111.30718) (width 0.25) (layer F.Cu) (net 5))
 (segment (start 165.01781 108.73) (end 162.56901 111.1788) (width 0.25) (layer F.Cu) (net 5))
 (segment (start 162.11619 111.76) (end 157.48 111.76) (width 0.25) (layer F.Cu) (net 5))
 (segment (start 176.276 108.73) (end 165.01781 108.73) (width 0.25) (layer F.Cu) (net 5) (status 10))
 (segment (start 157.48 111.76) (end 160.528 108.904) (width 0.25) (layer F.Cu) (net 5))
 (segment (start 155.64 113.792) (end 157.48 111.76) (width 0.25) (layer F.Cu) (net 5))
 (segment (start 140.208 111.76) (end 140.208 111.185) (width 0.25) (layer F.Cu) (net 7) (status 30))
 (segment (start 140.208 106.304) (end 140.076 106.172) (width 0.25) (layer F.Cu) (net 7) (status 30))
 (segment (start 140.208 111.76) (end 140.208 106.304) (width 0.25) (layer F.Cu) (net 7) (status 30))
 (segment (start 138.176 105.472) (end 138.176 106.172) (width 0.25) (layer F.Cu) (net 6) (status 20))
 (segment (start 140.968 102.68) (end 138.176 105.472) (width 0.25) (layer F.Cu) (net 6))
 (segment (start 143.764 102.68) (end 140.968 102.68) (width 0.25) (layer F.Cu) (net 6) (status 10))
 (segment (start 159.578 105.504) (end 159.578 106.204) (width 0.25) (layer F.Cu) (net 19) (status 20))
 (segment (start 156.754 102.68) (end 159.578 105.504) (width 0.25) (layer F.Cu) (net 19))
 (segment (start 153.924 102.68) (end 156.754 102.68) (width 0.25) (layer F.Cu) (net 19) (status 10))
 (segment (start 161.478 106.904) (end 161.478 106.204) (width 0.25) (layer F.Cu) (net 20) (status 20))
 (segment (start 161.544 106.27) (end 161.478 106.204) (width 0.25) (layer F.Cu) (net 20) (status 30))
 (segment (start 161.544 110.744) (end 161.544 106.27) (width 0.25) (layer F.Cu) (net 20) (status 30))
 (segment (start 123.462 114.3) (end 126.492 114.3) (width 0.25) (layer F.Cu) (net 10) (status 30))
 (segment (start 132.57 107.678) (end 134.62 107.678) (width 0.25) (layer F.Cu) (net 9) (status 20))
 (segment (start 131.572 106.68) (end 132.57 107.678) (width 0.25) (layer F.Cu) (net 9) (status 10))
 (segment (start 129.032 117.348) (end 129.032 114.3) (width 0.25) (layer F.Cu) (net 8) (status 30))
 (segment (start 167.098 113.284) (end 168.148 113.284) (width 0.25) (layer F.Cu) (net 4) (status 20))
 (segment (start 165.608 111.794) (end 167.098 113.284) (width 0.25) (layer F.Cu) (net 4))
 (segment (start 165.608 109.728) (end 165.608 111.794) (width 0.25) (layer F.Cu) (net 4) (status 10))
 (segment (start 176.276 106.105) (end 176.276 106.68) (width 0.25) (layer F.Cu) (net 3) (status 30))
 (segment (start 175.835 105.664) (end 176.276 106.105) (width 0.25) (layer F.Cu) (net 3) (status 20))
 (segment (start 173.228 105.664) (end 175.835 105.664) (width 0.25) (layer F.Cu) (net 3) (status 10))
 (segment (start 170.688 117.348) (end 170.688 113.284) (width 0.25) (layer F.Cu) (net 2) (status 30))
 (segment (start 143.764 111.252) (end 143.764 106.68) (width 0.25) (layer F.Cu) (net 22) (status 30))
 (segment (start 153.924 106.68) (end 143.764 106.68) (width 0.25) (layer F.Cu) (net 22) (status 30))
 (segment (start 144.939001 129.106999) (end 144.506 129.54) (width 0.25) (layer B.Cu) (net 22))
 (segment (start 144.506 129.54) (end 143.256 129.54) (width 0.25) (layer B.Cu) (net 22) (status 20))
 (segment (start 144.939001 112.427001) (end 144.939001 129.106999) (width 0.25) (layer B.Cu) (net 22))
 (segment (start 143.764 111.252) (end 144.939001 112.427001) (width 0.25) (layer B.Cu) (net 22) (status 10))
 (via (at 161.544 123.444) (size 0.8) (drill 0.4) (layers F.Cu B.Cu) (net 12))
 (segment (start 161.544 123.444) (end 161.544 112.794) (width 0.25) (layer F.Cu) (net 12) (status 20))
 (segment (start 146.144999 138.843001) (end 161.544 123.444) (width 0.25) (layer B.Cu) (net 12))
 (segment (start 134.563999 138.843001) (end 146.144999 138.843001) (width 0.25) (layer B.Cu) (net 12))
 (segment (start 133.952999 138.232001) (end 134.563999 138.843001) (width 0.25) (layer B.Cu) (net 12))
 (segment (start 133.952999 137.103999) (end 133.952999 138.232001) (width 0.25) (layer B.Cu) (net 12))
 (segment (start 137.256501 133.800497) (end 133.952999 137.103999) (width 0.25) (layer B.Cu) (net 12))
 (segment (start 137.256501 126.395499) (end 137.256501 133.800497) (width 0.25) (layer B.Cu) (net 12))
 (segment (start 138.684 124.968) (end 137.256501 126.395499) (width 0.25) (layer B.Cu) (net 12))
 (segment (start 122.13006 85.344) (end 129.032 78.44206) (width 1) (layer B.Cu) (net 15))
 (segment (start 119.38 85.344) (end 122.13006 85.344) (width 1) (layer B.Cu) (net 15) (status 10))
 (segment (start 177.58994 85.344) (end 170.434 78.18806) (width 1) (layer B.Cu) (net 15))
 (segment (start 180.34 85.344) (end 177.58994 85.344) (width 1) (layer B.Cu) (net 15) (status 10))
 (segment (start 129.032 78.44206) (end 129.032 75.184) (width 1) (layer B.Cu) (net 15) (status 20))
 (segment (start 170.434 78.18806) (end 170.434 75.184) (width 1) (layer B.Cu) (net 15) (status 20))
 (segment (start 170.434 77.93406) (end 170.434 75.184) (width 1) (layer B.Cu) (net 15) (status 20))
 (segment (start 169.926 78.44206) (end 170.434 77.93406) (width 1) (layer B.Cu) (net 15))
 (segment (start 129.032 78.44206) (end 169.926 78.44206) (width 1) (layer B.Cu) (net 15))
 (segment (start 141.624 83.82) (end 143.764 81.68) (width 1) (layer B.Cu) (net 18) (status 20))
 (segment (start 131.826 83.82) (end 141.624 83.82) (width 1) (layer B.Cu) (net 18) (status 10))
 (segment (start 137.624 97.82) (end 143.764 91.68) (width 1) (layer F.Cu) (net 16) (status 20))
 (segment (start 131.826 97.82) (end 137.624 97.82) (width 1) (layer F.Cu) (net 16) (status 10))
 (segment (start 156.064 83.82) (end 153.924 81.68) (width 1) (layer B.Cu) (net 23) (status 20))
 (segment (start 168.148 83.82) (end 156.064 83.82) (width 1) (layer B.Cu) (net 23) (status 10))
 (segment (start 160.064 97.82) (end 153.924 91.68) (width 1) (layer F.Cu) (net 24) (status 20))
 (segment (start 168.148 97.82) (end 160.064 97.82) (width 1) (layer F.Cu) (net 24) (status 10)))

